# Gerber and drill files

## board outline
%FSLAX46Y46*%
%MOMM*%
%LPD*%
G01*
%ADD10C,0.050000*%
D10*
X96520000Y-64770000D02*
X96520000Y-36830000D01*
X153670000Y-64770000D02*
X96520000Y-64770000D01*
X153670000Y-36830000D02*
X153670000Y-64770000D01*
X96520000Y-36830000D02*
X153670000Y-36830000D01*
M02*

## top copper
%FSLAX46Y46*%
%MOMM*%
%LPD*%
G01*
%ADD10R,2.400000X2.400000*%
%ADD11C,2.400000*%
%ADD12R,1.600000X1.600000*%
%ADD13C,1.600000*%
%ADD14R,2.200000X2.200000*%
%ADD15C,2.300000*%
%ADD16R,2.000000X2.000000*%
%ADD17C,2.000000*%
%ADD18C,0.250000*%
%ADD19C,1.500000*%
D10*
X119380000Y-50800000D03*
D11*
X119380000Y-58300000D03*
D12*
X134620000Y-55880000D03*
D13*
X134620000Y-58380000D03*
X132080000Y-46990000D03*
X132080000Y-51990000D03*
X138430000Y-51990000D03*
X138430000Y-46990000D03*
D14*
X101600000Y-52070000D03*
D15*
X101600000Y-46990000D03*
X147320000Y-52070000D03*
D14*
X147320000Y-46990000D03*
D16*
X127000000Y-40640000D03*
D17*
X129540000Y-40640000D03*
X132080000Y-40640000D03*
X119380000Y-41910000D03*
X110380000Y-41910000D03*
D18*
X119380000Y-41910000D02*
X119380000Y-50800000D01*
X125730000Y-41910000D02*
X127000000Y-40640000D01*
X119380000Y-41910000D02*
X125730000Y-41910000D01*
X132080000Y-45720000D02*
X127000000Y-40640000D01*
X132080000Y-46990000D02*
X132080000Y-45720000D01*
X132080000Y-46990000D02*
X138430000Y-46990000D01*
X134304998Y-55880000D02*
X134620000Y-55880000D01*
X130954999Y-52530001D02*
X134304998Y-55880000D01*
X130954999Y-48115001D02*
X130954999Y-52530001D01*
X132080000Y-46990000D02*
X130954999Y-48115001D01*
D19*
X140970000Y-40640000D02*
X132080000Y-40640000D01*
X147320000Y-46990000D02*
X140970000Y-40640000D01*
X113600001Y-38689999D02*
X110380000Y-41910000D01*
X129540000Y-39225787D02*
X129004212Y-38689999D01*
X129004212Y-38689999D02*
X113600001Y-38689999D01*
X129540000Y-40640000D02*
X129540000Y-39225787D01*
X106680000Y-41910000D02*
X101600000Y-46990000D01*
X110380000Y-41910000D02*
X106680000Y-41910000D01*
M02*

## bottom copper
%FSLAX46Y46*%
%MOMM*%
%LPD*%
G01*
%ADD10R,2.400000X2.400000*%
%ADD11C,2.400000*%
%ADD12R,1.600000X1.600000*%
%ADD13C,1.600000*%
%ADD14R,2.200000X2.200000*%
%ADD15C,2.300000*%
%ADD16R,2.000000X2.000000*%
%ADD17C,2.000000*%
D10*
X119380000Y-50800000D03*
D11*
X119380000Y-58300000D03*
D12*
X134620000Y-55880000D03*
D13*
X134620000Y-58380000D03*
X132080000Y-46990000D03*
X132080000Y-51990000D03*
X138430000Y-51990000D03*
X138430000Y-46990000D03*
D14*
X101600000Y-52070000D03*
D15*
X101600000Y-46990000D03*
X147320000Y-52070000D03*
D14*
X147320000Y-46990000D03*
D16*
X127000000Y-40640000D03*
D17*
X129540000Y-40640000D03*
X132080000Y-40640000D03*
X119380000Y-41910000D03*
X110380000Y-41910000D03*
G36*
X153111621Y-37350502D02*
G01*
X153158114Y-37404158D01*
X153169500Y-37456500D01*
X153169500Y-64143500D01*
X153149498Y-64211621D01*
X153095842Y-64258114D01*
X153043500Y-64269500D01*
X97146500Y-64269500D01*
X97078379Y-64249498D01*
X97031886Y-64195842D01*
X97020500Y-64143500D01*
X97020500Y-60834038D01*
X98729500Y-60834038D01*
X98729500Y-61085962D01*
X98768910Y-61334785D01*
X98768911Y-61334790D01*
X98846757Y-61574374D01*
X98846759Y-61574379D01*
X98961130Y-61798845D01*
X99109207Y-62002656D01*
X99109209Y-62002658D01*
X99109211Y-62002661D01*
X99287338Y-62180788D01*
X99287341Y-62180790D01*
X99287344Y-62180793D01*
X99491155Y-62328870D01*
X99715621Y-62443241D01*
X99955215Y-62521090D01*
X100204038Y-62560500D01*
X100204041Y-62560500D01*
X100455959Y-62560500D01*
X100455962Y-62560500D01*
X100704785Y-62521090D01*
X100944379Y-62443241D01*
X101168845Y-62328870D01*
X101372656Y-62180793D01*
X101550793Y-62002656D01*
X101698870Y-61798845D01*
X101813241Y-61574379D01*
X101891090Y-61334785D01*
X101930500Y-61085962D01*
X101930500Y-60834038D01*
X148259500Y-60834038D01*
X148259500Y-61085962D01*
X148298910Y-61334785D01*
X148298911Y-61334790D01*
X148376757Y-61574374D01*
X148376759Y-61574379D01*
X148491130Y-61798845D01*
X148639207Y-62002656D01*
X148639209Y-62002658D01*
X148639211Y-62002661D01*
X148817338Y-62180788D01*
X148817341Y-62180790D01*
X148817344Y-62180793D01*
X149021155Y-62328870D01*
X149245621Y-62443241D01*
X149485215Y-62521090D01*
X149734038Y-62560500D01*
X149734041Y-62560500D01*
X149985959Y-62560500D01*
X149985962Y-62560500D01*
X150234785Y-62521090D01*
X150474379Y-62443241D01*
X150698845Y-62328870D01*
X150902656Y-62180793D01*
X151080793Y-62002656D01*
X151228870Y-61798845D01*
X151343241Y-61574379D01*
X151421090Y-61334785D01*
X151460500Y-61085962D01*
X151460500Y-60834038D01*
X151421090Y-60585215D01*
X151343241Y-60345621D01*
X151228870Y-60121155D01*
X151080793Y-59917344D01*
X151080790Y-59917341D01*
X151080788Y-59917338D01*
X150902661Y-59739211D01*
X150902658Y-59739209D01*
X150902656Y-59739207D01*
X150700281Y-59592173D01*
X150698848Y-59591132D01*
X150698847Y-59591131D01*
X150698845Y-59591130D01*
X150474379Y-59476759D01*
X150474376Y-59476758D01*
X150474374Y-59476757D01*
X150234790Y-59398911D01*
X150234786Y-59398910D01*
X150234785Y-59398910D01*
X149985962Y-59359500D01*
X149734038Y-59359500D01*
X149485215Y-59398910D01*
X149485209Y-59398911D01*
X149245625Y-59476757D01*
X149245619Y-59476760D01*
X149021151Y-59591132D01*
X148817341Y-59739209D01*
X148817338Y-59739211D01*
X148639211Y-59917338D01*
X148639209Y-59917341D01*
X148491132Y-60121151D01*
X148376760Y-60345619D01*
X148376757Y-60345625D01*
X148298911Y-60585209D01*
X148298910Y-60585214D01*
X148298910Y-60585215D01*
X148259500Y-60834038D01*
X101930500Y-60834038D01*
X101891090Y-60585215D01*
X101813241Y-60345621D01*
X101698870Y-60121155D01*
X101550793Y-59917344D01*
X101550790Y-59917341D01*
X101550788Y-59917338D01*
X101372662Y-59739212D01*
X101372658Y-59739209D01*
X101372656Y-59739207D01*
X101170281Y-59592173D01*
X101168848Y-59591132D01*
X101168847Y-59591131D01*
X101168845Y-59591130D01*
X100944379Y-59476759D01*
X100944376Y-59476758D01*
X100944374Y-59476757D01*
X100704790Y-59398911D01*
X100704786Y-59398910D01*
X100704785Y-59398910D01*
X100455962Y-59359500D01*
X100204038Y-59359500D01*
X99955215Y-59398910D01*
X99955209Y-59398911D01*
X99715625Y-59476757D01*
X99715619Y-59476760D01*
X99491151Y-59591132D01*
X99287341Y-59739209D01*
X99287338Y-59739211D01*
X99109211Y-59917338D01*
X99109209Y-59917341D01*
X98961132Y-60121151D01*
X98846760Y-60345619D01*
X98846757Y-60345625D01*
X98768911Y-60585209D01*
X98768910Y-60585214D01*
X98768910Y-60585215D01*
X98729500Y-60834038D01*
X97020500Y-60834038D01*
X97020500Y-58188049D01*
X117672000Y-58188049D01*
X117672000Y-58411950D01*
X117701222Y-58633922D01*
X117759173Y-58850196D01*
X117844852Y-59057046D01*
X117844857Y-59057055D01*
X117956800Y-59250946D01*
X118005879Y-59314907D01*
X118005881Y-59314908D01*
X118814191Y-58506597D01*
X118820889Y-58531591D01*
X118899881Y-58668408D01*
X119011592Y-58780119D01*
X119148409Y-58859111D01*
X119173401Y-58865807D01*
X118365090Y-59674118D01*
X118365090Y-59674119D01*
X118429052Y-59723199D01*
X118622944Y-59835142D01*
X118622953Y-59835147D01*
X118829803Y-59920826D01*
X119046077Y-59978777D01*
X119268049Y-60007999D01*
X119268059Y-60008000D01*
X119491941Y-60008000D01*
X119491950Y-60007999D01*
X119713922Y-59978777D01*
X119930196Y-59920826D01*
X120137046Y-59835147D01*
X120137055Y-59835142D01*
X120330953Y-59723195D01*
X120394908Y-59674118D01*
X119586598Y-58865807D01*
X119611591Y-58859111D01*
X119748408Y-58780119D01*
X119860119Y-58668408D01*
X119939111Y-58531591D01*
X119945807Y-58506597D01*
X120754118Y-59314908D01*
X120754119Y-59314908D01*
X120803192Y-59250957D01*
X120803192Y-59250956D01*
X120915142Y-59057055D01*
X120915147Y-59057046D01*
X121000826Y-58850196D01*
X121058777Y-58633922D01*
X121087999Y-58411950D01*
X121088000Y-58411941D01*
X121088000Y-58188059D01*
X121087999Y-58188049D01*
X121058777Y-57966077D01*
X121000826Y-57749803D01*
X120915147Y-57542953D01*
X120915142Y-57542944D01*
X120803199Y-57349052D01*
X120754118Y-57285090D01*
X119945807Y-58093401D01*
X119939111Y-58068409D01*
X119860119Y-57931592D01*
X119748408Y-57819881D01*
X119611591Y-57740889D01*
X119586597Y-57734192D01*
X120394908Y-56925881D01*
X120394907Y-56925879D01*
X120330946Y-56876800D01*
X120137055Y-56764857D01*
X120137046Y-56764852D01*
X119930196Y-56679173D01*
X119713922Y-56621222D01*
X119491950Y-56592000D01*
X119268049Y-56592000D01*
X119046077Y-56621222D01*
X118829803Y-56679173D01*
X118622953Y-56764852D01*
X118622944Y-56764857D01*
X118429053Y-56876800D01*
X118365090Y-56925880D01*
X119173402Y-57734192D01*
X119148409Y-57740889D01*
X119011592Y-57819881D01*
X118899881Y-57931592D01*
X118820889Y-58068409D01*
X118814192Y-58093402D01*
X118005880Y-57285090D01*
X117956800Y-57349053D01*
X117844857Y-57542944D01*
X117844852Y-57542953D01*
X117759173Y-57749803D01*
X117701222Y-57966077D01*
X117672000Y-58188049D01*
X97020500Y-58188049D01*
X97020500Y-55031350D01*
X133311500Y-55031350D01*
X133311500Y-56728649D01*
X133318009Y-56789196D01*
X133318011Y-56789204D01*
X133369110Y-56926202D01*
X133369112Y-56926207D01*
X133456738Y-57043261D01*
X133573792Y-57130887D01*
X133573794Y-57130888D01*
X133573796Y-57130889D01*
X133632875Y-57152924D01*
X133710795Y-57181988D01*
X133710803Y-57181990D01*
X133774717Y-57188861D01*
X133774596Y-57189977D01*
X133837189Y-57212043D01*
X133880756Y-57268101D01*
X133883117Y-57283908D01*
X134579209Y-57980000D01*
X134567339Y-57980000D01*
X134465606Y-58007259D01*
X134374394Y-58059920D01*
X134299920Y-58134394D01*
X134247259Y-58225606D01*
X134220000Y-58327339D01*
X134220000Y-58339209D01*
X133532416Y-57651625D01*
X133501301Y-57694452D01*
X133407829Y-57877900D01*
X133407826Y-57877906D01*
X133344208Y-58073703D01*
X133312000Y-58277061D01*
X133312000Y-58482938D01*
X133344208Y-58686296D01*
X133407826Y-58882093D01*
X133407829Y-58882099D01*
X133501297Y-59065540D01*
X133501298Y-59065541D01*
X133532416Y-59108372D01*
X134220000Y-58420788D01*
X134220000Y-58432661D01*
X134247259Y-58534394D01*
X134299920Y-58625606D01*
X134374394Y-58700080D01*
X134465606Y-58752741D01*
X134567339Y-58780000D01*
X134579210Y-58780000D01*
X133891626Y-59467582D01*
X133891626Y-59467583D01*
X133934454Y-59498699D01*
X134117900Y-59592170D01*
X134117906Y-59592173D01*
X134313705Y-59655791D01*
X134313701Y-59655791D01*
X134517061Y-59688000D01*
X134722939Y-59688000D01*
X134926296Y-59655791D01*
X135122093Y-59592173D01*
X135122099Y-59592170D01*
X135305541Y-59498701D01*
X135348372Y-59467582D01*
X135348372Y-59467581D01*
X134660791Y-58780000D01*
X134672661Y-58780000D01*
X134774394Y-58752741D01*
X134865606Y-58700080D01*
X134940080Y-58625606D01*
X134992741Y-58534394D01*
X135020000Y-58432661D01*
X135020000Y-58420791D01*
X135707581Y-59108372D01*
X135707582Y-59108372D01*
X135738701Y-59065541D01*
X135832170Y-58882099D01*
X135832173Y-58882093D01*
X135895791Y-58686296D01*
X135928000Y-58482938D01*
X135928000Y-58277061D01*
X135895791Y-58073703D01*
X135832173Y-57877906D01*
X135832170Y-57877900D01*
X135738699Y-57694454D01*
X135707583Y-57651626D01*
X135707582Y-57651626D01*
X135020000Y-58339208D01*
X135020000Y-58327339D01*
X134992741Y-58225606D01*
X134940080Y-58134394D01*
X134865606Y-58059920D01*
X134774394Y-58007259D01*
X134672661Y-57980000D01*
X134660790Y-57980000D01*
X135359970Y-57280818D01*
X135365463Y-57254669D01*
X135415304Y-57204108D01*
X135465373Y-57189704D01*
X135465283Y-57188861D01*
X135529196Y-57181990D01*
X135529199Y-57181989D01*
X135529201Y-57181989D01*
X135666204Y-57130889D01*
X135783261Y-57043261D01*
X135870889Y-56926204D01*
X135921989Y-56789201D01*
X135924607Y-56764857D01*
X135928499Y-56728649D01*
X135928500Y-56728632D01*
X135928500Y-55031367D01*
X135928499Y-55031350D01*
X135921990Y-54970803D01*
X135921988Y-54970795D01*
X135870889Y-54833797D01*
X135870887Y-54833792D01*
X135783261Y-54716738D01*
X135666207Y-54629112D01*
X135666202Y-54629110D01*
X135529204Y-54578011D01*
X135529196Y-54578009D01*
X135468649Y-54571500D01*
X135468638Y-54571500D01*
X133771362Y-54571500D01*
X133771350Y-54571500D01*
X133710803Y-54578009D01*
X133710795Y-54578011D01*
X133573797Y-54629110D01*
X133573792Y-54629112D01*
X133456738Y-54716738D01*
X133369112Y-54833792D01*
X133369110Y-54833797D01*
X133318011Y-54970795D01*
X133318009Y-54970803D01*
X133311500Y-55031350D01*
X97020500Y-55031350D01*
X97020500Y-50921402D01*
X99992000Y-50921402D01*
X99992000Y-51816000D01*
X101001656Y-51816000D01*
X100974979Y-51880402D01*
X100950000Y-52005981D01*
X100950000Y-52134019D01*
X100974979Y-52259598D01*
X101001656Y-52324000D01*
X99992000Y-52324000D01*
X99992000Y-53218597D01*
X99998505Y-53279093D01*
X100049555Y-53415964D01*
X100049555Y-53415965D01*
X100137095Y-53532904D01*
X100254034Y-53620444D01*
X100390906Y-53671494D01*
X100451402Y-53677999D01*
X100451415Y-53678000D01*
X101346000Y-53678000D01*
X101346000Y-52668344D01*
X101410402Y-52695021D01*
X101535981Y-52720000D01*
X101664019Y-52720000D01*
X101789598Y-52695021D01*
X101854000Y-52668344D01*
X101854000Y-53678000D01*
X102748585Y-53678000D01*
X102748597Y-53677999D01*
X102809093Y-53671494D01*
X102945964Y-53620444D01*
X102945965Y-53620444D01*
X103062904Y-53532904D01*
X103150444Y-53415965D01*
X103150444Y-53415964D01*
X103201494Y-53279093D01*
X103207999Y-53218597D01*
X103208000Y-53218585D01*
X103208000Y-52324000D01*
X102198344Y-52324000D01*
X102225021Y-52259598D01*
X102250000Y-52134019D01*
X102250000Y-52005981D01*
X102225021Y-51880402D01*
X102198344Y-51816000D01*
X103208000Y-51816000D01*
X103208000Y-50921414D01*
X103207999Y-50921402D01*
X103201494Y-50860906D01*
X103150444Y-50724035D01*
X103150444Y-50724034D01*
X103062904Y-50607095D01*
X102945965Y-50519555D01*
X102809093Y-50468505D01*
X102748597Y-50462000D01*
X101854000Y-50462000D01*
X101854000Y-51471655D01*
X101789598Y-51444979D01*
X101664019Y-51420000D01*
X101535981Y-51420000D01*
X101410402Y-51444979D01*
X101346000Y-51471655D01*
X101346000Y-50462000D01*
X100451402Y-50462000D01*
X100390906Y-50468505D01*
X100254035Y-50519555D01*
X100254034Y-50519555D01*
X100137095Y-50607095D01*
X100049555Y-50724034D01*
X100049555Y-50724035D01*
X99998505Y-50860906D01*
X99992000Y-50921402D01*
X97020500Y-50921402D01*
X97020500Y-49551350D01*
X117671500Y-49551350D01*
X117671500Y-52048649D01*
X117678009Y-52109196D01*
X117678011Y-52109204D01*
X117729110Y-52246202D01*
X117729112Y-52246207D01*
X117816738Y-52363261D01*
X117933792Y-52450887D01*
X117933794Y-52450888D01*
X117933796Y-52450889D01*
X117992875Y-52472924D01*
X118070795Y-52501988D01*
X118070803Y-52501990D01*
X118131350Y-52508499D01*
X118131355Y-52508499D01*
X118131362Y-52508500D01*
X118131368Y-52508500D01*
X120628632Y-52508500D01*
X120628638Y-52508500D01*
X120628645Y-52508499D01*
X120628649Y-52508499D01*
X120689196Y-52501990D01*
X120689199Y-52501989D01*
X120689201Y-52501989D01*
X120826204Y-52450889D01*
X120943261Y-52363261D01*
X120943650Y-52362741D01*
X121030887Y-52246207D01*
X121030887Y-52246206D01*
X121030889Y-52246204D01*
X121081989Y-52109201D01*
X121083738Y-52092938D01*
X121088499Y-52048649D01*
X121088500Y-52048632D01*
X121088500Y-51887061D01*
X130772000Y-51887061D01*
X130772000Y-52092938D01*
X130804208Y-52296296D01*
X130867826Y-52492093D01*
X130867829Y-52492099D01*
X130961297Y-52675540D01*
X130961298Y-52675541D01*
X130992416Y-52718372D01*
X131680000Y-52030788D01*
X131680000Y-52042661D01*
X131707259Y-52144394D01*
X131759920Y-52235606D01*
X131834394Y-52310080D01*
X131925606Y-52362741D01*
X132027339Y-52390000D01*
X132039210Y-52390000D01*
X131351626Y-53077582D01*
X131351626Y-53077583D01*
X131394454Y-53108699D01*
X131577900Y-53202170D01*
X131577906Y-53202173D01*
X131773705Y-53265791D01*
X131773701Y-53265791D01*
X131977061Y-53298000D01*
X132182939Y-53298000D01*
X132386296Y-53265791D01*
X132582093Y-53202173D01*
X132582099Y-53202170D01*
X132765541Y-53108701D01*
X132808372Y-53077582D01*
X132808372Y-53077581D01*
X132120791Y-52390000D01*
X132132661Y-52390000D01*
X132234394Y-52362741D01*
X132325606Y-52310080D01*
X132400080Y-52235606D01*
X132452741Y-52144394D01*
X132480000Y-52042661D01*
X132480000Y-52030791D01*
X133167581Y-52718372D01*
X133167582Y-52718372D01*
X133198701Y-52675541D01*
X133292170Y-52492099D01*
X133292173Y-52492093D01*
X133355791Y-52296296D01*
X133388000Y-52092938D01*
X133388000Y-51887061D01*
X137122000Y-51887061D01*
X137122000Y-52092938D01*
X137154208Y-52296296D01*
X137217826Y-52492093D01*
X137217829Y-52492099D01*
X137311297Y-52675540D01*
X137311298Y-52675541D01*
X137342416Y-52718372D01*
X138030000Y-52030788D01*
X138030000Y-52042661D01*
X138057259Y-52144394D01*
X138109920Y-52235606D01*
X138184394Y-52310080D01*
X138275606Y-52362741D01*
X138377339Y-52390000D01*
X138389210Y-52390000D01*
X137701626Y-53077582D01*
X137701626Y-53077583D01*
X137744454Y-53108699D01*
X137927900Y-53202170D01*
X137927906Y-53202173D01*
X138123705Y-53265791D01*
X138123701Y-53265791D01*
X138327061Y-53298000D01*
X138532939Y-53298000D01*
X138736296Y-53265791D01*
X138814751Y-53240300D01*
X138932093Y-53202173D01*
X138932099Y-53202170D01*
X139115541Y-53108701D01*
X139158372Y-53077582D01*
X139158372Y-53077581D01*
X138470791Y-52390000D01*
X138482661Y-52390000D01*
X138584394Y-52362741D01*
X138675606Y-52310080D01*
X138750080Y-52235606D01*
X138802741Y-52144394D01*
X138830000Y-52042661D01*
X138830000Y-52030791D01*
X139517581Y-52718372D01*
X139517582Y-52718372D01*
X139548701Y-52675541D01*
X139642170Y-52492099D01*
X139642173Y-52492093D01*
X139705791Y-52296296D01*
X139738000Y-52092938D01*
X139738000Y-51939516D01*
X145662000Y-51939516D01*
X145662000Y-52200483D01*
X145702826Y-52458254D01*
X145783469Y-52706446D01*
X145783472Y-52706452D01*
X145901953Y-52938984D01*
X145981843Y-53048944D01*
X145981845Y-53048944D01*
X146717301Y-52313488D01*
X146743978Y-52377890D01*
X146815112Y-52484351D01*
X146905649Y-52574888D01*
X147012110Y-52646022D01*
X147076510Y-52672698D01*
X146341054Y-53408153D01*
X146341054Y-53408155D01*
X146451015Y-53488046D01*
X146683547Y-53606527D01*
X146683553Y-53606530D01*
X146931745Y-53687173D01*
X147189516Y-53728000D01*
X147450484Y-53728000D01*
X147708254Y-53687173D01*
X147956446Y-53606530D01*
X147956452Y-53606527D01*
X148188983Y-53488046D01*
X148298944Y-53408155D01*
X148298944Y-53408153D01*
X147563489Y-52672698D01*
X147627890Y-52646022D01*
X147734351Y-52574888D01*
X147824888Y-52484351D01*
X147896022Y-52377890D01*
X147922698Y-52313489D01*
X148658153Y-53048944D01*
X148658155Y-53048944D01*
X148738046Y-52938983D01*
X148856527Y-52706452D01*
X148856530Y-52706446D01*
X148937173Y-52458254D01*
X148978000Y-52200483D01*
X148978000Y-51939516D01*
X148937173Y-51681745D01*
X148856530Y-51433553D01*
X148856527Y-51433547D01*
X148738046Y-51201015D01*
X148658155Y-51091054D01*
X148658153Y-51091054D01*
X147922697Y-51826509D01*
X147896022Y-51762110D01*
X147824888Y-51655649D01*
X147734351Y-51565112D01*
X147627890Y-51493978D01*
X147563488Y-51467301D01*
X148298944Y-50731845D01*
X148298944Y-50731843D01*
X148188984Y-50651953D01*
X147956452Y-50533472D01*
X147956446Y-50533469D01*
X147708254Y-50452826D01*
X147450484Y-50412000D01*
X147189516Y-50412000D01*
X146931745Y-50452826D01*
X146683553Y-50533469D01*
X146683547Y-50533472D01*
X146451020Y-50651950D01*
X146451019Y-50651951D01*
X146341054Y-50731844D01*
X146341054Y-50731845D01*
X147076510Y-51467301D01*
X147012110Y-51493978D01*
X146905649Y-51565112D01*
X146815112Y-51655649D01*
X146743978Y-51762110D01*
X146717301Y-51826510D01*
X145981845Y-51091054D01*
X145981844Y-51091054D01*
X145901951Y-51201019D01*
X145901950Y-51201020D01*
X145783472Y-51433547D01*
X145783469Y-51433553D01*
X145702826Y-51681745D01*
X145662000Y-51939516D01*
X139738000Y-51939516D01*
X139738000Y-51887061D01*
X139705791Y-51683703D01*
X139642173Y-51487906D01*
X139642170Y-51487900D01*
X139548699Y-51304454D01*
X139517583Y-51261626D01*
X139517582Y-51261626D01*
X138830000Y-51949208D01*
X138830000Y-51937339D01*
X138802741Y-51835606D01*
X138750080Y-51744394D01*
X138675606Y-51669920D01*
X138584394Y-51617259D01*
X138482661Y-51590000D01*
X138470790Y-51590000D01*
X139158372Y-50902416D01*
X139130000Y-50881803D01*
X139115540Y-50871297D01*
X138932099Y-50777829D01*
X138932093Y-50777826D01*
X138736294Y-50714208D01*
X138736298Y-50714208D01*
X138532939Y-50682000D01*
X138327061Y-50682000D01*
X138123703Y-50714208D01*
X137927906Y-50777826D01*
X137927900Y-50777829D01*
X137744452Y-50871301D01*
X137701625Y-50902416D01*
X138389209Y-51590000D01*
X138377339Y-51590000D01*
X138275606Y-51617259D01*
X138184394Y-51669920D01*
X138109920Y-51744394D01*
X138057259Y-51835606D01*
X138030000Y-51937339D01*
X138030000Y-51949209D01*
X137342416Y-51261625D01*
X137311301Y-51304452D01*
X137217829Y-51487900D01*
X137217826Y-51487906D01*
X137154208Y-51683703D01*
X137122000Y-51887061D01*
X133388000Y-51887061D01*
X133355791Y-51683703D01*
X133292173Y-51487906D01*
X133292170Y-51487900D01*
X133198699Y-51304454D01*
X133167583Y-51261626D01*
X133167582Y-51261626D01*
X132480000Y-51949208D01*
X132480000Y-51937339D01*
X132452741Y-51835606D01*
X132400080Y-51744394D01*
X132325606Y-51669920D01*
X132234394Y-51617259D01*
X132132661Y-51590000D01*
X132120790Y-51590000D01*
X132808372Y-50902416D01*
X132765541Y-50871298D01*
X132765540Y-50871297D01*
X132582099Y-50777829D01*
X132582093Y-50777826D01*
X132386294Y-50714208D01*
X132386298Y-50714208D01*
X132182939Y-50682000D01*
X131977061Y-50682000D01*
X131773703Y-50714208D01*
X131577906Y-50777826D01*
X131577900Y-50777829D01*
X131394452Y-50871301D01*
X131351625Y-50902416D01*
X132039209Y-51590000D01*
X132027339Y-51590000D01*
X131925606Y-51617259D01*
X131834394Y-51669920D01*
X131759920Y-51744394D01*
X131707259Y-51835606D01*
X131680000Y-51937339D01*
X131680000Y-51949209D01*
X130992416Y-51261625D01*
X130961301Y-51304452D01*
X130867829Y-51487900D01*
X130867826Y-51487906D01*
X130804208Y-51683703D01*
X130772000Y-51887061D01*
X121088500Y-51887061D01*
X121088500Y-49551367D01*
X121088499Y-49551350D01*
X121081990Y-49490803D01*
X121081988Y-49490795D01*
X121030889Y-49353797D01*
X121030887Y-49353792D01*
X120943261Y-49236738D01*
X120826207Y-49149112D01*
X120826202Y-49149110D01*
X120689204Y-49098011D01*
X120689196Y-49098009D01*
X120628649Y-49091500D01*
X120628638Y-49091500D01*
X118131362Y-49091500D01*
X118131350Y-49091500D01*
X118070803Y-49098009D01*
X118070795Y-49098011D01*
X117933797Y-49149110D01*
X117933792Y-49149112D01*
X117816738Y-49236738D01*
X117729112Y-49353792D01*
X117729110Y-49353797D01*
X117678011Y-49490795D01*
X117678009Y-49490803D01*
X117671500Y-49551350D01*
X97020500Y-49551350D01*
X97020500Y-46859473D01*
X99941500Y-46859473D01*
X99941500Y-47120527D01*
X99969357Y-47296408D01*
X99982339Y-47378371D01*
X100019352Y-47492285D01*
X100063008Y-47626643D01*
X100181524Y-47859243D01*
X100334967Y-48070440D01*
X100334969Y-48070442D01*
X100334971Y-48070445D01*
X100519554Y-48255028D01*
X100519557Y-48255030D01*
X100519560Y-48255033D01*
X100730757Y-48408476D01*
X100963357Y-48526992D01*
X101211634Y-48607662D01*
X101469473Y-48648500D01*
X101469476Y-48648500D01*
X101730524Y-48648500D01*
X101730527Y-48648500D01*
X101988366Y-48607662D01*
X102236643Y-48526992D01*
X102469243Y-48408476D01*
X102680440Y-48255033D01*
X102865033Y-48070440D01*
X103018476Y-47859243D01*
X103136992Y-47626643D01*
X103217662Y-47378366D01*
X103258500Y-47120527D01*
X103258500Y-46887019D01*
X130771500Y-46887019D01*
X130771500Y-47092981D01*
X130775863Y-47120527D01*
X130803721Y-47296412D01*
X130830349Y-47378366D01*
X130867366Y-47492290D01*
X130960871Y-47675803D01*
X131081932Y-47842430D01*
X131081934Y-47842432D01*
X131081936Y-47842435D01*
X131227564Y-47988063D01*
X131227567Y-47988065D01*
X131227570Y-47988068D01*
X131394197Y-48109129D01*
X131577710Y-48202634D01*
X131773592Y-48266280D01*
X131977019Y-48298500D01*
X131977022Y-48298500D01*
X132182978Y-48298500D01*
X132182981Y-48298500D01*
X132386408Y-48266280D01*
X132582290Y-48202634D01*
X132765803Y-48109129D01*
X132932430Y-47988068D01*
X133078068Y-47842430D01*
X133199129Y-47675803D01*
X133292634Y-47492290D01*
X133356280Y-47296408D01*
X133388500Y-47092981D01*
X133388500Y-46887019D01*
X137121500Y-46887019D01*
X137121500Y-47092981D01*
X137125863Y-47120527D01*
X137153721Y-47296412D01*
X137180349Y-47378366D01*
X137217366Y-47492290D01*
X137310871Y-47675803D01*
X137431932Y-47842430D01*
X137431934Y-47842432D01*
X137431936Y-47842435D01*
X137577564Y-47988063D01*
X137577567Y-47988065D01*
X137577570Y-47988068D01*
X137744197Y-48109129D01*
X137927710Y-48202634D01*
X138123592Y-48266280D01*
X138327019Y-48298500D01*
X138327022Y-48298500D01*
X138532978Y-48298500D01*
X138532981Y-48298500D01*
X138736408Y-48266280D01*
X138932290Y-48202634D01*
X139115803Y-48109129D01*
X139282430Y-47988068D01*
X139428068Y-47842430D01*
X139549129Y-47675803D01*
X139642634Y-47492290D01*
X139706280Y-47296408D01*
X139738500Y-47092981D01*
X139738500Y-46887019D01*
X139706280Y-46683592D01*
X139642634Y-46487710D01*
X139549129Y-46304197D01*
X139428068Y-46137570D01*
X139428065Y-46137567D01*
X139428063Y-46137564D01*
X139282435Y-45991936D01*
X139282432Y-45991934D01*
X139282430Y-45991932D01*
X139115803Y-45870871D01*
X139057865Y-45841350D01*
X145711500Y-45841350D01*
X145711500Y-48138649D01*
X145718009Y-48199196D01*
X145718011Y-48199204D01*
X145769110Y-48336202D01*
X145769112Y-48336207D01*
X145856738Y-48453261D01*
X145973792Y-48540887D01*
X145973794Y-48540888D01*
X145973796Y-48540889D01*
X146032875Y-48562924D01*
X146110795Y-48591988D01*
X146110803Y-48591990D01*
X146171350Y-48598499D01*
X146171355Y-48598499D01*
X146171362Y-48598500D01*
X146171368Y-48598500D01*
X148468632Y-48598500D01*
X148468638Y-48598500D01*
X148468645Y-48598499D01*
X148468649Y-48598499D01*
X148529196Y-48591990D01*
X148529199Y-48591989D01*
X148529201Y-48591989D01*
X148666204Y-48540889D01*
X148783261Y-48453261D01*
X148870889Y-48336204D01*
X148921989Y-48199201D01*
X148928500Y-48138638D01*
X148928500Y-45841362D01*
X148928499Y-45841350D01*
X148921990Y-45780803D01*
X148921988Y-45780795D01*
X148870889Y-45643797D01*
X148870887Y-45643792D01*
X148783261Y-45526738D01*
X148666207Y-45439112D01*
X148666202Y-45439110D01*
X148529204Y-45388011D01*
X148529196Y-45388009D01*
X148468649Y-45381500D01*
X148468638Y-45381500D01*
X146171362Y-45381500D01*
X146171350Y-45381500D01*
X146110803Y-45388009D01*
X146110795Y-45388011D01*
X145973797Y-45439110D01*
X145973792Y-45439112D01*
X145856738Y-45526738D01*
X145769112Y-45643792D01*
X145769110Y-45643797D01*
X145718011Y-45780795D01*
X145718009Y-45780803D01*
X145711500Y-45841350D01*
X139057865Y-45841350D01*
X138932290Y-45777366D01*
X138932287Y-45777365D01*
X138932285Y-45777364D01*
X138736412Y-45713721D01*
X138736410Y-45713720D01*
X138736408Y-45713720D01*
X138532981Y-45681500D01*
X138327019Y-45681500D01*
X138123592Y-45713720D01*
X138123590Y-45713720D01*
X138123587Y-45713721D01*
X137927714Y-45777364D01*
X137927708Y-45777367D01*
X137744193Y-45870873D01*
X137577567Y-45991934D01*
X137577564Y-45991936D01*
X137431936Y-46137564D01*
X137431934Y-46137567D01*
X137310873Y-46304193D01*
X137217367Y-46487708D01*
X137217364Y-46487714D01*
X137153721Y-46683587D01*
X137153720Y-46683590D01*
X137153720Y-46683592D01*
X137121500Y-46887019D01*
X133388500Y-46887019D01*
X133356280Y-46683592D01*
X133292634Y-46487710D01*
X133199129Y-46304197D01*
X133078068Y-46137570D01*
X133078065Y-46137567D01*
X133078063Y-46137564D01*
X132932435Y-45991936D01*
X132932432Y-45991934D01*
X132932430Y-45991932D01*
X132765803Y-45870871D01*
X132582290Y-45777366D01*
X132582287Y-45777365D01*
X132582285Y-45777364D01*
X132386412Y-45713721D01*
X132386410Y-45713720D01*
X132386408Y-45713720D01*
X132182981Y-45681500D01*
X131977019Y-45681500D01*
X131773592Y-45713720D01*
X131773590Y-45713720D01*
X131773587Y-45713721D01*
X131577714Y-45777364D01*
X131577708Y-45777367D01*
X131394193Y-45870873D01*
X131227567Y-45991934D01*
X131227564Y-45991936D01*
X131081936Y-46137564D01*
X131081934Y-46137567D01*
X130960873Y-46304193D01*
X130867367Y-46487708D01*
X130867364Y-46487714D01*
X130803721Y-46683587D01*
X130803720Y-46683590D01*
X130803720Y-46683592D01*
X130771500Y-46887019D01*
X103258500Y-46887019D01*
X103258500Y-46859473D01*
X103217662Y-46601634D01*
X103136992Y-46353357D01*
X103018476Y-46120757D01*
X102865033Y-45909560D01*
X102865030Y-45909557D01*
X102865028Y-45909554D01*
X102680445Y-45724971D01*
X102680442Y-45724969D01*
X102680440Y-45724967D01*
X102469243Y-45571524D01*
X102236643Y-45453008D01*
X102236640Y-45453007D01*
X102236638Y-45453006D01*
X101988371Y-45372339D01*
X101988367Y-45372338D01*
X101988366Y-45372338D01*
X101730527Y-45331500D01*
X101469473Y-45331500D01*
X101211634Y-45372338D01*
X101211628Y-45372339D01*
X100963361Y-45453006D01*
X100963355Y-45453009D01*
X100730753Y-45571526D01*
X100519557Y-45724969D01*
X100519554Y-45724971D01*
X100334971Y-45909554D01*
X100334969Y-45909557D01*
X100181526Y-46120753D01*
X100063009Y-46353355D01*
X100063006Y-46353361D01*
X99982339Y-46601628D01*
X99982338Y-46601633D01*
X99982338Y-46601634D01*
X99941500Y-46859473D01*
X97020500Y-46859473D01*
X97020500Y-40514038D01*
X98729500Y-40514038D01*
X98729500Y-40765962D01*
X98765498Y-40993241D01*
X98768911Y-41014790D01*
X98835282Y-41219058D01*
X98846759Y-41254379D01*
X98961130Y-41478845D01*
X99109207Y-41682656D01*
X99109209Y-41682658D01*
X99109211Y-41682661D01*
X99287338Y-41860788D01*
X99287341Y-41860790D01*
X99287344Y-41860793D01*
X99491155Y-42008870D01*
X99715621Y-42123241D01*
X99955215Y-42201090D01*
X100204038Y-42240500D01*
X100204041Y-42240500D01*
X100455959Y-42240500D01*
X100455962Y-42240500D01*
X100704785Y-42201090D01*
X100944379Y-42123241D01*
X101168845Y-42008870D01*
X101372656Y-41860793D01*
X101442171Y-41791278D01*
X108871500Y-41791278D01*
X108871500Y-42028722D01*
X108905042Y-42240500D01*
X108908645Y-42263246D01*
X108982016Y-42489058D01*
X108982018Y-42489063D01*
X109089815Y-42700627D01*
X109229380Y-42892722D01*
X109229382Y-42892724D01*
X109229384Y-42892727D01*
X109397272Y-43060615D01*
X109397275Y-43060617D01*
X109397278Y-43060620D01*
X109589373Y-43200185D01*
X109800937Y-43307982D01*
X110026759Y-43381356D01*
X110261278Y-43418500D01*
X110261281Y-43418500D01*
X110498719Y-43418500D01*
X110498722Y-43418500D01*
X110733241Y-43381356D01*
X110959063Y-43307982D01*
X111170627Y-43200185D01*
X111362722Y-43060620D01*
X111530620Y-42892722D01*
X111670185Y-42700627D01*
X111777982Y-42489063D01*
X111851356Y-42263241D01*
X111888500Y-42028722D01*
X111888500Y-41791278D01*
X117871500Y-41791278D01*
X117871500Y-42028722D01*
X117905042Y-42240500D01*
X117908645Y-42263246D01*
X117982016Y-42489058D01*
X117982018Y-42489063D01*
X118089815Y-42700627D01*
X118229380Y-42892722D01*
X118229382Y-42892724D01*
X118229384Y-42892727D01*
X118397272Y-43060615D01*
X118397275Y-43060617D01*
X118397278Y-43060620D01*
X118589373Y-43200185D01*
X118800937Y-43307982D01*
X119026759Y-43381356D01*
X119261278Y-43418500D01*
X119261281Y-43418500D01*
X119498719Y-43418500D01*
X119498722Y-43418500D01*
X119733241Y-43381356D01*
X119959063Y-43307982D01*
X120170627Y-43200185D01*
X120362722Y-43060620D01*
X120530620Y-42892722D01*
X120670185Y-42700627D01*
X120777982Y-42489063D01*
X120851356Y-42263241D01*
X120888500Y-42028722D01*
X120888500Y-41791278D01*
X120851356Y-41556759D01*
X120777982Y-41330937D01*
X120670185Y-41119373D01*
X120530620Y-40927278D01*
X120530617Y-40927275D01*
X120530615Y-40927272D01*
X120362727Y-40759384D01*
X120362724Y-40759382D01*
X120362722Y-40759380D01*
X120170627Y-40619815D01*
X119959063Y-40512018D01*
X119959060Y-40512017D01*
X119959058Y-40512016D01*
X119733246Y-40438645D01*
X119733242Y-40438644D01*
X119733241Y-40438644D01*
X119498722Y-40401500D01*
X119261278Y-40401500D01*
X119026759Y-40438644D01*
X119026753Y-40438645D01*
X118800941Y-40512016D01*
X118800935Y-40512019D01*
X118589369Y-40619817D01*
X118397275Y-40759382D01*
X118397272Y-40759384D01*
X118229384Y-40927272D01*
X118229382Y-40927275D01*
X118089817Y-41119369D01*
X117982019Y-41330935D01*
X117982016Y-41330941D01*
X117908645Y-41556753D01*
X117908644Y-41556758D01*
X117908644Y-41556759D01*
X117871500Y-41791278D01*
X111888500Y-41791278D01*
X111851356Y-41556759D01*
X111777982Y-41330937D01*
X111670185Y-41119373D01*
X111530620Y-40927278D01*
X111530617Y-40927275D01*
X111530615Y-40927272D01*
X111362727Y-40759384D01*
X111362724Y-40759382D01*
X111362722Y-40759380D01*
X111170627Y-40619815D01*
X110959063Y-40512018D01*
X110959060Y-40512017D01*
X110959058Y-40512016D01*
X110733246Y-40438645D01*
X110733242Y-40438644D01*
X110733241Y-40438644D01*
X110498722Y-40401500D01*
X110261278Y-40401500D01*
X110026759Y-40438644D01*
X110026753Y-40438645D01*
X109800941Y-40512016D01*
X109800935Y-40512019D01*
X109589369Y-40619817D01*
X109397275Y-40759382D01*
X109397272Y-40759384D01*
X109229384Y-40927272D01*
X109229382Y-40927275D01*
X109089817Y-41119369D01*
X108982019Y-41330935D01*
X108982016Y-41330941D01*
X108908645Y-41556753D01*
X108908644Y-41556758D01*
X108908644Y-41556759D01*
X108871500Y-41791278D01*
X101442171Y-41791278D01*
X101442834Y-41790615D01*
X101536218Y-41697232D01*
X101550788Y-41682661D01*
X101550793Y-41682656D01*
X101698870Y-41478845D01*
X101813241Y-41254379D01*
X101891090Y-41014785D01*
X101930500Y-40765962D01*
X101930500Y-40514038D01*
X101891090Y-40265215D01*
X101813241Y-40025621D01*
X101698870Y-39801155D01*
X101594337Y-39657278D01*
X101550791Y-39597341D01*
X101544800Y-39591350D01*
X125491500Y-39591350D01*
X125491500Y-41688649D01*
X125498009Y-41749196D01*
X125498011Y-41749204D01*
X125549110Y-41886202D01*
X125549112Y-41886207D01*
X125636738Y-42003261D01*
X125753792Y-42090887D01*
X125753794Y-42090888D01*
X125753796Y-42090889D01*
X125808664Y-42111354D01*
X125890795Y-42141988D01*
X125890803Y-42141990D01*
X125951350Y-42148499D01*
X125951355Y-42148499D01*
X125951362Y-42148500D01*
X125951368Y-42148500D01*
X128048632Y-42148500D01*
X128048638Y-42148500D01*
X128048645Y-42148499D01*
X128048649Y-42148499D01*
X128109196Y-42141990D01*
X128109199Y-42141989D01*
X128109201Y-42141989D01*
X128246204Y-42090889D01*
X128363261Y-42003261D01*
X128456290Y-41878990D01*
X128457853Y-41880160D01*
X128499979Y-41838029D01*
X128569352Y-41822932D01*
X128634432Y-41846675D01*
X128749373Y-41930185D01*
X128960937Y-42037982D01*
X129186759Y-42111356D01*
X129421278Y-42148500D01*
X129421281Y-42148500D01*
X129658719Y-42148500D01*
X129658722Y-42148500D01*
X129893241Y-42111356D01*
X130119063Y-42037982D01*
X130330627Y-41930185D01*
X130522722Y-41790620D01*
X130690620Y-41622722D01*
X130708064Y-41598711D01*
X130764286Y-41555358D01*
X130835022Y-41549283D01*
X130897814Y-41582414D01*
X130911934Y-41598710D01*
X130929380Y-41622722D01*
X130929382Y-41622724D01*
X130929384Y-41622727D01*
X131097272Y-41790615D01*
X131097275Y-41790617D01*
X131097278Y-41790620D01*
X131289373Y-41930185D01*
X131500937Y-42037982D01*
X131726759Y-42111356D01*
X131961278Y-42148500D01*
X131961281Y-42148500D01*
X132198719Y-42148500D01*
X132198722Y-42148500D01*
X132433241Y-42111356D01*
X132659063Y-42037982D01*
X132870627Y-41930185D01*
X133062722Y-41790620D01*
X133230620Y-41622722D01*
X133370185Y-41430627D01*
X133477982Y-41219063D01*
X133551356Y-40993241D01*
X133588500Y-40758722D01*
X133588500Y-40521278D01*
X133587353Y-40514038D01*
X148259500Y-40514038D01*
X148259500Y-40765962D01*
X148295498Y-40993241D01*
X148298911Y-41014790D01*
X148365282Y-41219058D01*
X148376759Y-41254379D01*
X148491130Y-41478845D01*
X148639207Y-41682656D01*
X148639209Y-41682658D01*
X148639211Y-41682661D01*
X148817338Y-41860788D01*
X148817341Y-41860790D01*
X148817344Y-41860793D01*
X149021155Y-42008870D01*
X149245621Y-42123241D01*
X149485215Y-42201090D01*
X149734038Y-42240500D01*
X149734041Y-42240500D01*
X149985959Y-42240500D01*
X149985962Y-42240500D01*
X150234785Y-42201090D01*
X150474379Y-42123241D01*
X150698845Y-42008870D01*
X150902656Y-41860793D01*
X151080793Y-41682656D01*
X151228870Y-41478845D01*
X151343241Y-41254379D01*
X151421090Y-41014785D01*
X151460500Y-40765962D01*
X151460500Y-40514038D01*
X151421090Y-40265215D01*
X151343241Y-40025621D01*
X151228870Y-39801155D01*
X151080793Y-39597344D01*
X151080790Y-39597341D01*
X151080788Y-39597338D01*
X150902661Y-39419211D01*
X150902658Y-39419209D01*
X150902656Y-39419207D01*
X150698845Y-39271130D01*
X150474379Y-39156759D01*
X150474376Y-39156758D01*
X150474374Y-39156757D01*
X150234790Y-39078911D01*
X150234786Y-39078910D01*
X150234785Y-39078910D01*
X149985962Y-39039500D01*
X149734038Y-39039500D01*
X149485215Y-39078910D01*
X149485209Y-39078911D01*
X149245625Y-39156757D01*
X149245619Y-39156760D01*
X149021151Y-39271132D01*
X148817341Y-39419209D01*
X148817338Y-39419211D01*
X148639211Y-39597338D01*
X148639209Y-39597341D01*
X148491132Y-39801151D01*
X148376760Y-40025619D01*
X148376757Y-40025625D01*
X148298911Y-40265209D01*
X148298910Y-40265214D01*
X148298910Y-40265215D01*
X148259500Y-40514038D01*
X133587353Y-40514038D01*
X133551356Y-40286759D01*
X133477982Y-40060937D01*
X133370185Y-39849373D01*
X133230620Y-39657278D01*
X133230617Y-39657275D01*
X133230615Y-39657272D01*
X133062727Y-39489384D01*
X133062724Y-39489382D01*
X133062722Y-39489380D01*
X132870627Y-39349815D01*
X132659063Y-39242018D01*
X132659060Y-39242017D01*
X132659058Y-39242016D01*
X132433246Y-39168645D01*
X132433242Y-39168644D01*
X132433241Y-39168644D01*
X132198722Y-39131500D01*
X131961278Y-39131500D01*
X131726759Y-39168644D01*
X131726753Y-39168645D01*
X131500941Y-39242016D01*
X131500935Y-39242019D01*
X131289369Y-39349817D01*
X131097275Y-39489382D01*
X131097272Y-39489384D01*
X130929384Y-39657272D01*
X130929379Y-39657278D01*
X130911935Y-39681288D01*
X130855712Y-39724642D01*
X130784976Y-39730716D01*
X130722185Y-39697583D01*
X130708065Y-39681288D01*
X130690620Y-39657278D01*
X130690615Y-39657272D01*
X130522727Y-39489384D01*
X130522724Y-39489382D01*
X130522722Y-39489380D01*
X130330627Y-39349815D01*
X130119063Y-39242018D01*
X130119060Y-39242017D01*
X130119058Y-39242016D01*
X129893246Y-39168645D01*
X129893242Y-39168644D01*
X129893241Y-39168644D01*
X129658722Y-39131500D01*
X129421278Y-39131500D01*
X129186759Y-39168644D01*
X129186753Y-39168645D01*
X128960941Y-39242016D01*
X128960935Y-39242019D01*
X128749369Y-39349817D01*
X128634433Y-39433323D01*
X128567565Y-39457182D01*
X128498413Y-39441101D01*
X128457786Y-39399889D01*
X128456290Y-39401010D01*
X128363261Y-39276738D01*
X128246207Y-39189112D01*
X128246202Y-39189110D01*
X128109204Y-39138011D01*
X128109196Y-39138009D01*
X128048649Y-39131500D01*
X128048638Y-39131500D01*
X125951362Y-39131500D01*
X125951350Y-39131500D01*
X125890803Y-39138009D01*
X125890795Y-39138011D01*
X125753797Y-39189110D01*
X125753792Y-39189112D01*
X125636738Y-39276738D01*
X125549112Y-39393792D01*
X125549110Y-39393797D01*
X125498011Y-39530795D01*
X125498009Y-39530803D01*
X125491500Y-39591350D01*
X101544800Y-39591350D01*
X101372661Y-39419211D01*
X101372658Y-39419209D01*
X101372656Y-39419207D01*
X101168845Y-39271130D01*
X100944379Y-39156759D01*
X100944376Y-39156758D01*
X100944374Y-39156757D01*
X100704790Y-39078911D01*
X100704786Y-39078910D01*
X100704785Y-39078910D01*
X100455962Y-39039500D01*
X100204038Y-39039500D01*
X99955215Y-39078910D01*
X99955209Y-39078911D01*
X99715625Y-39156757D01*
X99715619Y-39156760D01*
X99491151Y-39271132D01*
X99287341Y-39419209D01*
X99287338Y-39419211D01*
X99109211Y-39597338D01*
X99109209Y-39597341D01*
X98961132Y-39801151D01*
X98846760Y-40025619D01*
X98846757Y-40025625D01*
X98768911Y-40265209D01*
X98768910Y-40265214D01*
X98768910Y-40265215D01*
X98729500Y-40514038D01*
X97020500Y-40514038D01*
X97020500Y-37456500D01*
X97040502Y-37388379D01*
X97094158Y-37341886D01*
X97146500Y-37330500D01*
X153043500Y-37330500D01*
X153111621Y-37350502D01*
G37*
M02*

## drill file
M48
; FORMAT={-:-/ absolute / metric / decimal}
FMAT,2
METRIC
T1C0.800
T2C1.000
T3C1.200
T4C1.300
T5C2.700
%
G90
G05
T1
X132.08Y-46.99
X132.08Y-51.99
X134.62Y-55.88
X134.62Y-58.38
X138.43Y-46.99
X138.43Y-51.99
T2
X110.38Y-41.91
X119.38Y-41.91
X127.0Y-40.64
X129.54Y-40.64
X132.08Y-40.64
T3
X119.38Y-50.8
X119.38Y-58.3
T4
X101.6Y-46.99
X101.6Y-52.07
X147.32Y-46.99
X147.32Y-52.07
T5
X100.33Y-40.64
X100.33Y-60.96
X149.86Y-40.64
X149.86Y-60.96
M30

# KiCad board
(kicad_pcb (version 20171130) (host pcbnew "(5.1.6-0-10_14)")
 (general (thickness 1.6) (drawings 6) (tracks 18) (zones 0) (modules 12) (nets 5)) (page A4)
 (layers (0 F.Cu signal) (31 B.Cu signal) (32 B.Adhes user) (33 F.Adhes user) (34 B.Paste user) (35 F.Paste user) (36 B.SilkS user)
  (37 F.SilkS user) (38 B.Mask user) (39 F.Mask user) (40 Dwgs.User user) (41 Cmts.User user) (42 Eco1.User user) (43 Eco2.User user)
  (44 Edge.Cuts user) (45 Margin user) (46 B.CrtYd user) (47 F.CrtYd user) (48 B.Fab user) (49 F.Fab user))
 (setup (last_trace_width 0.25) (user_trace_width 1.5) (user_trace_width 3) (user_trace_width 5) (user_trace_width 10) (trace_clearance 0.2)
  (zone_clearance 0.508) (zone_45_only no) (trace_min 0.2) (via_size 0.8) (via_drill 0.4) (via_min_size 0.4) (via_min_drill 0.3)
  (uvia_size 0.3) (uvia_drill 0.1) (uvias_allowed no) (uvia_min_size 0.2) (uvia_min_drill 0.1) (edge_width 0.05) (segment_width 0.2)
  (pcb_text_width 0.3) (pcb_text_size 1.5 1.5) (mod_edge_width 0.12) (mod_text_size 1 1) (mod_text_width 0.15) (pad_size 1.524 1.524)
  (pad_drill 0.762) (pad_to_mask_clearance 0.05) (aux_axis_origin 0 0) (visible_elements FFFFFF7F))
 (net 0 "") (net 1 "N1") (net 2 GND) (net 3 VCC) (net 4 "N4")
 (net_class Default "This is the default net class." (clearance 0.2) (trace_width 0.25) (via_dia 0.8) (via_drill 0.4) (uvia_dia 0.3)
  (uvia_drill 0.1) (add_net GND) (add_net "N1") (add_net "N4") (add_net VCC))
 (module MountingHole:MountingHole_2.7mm (layer F.Cu) (at 149.86 60.96)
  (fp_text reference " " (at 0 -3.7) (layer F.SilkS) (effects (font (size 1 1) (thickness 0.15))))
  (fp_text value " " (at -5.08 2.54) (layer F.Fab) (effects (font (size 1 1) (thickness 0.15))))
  (pad 1 np_thru_hole circle (at 0 0) (size 2.7 2.7) (drill 2.7) (layers *.Cu *.Mask)))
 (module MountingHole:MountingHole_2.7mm (layer F.Cu) (at 149.86 40.64)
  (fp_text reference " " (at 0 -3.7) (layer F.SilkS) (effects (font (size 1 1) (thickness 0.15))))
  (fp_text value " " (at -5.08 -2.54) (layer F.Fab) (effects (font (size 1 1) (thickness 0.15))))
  (pad 1 np_thru_hole circle (at 0 0) (size 2.7 2.7) (drill 2.7) (layers *.Cu *.Mask)))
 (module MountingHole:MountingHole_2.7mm (layer F.Cu) (at 100.33 60.96)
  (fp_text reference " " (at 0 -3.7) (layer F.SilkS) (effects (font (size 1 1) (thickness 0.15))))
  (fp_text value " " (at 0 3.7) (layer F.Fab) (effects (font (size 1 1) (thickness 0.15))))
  (pad 1 np_thru_hole circle (at 0 0) (size 2.7 2.7) (drill 2.7) (layers *.Cu *.Mask)))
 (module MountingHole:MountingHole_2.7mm (layer F.Cu) (at 100.33 40.64)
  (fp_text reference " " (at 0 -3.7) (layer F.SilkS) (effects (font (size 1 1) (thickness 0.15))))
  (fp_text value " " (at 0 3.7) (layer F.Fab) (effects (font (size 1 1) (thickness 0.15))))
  (pad 1 np_thru_hole circle (at 0 0) (size 2.7 2.7) (drill 2.7) (layers *.Cu *.Mask)))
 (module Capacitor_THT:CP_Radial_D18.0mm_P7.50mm (layer F.Cu) (at 119.38 50.8 270)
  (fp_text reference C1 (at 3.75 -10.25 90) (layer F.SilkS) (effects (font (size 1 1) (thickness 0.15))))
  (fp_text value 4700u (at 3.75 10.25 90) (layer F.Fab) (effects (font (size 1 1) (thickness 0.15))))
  (pad 1 thru_hole rect (at 0 0 270) (size 2.4 2.4) (drill 1.2) (layers *.Cu *.Mask) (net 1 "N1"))
  (pad 2 thru_hole circle (at 7.5 0 270) (size 2.4 2.4) (drill 1.2) (layers *.Cu *.Mask) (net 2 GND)))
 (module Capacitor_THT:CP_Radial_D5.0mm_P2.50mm (layer F.Cu) (at 134.62 55.88 270)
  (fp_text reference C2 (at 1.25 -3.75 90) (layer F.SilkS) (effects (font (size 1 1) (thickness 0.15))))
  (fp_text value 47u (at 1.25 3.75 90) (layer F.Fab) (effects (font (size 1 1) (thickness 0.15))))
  (pad 1 thru_hole rect (at 0 0 270) (size 1.6 1.6) (drill 0.8) (layers *.Cu *.Mask) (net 1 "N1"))
  (pad 2 thru_hole circle (at 2.5 0 270) (size 1.6 1.6) (drill 0.8) (layers *.Cu *.Mask) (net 2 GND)))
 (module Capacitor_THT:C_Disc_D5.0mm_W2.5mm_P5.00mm (layer F.Cu) (at 132.08 46.99 270)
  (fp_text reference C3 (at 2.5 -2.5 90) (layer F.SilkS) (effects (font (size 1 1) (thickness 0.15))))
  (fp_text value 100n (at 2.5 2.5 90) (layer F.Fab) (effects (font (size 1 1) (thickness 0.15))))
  (pad 1 thru_hole circle (at 0 0 270) (size 1.6 1.6) (drill 0.8) (layers *.Cu *.Mask) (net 1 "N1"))
  (pad 2 thru_hole circle (at 5 0 270) (size 1.6 1.6) (drill 0.8) (layers *.Cu *.Mask) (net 2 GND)))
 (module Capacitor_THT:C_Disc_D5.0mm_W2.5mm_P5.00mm (layer F.Cu) (at 138.43 46.99 270)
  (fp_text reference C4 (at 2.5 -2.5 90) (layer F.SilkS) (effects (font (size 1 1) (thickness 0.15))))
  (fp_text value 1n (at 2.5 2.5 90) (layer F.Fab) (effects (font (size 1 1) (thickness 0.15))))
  (pad 2 thru_hole circle (at 5 0 270) (size 1.6 1.6) (drill 0.8) (layers *.Cu *.Mask) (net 2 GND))
  (pad 1 thru_hole circle (at 0 0 270) (size 1.6 1.6) (drill 0.8) (layers *.Cu *.Mask) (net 1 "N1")))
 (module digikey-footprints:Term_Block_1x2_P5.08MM (layer F.Cu) (at 101.6 52.07 90)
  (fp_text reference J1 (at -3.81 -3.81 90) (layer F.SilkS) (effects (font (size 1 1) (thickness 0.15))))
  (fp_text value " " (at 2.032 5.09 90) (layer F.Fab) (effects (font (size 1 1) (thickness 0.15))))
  (pad 1 thru_hole rect (at 0 0 90) (size 2.2 2.2) (drill 1.3) (layers *.Cu *.Mask) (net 2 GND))
  (pad 2 thru_hole circle (at 5.08 0 90) (size 2.3 2.3) (drill 1.3) (layers *.Cu *.Mask) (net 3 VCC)))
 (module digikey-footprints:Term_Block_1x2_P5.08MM (layer F.Cu) (at 147.32 46.99 270)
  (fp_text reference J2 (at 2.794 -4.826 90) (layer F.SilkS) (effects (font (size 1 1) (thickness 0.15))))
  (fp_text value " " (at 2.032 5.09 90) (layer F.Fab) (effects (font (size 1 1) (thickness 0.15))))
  (pad 2 thru_hole circle (at 5.08 0 270) (size 2.3 2.3) (drill 1.3) (layers *.Cu *.Mask) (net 2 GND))
  (pad 1 thru_hole rect (at 0 0 270) (size 2.2 2.2) (drill 1.3) (layers *.Cu *.Mask) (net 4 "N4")))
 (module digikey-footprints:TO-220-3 (layer F.Cu) (at 127 40.64)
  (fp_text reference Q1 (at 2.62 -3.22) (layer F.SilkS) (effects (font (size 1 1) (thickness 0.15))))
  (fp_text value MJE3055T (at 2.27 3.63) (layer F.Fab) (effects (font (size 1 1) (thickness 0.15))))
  (pad 1 thru_hole rect (at 0 0) (size 2 2) (drill 1) (layers *.Cu *.Mask) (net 1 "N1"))
  (pad 2 thru_hole circle (at 2.54 0) (size 2 2) (drill 1) (layers *.Cu *.Mask) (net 3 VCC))
  (pad 3 thru_hole circle (at 5.08 0) (size 2 2) (drill 1) (layers *.Cu *.Mask) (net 4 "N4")))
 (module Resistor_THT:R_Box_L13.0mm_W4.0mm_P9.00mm (layer F.Cu) (at 119.38 41.91 180)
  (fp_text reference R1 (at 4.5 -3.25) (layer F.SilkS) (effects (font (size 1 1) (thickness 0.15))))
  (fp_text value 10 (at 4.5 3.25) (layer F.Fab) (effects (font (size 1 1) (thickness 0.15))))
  (pad 1 thru_hole circle (at 0 0 180) (size 2 2) (drill 1) (layers *.Cu *.Mask) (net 1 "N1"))
  (pad 2 thru_hole circle (at 9 0 180) (size 2 2) (drill 1) (layers *.Cu *.Mask) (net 3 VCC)))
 (gr_line (start 96.52 64.77) (end 96.52 36.83) (layer Edge.Cuts) (width 0.05))
 (gr_line (start 153.67 64.77) (end 96.52 64.77) (layer Edge.Cuts) (width 0.05))
 (gr_line (start 153.67 36.83) (end 153.67 64.77) (layer Edge.Cuts) (width 0.05))
 (gr_line (start 96.52 36.83) (end 153.67 36.83) (layer Edge.Cuts) (width 0.05))
 (segment (start 119.38 41.91) (end 119.38 50.8) (width 0.25) (layer F.Cu) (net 1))
 (segment (start 125.73 41.91) (end 127 40.64) (width 0.25) (layer F.Cu) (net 1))
 (segment (start 119.38 41.91) (end 125.73 41.91) (width 0.25) (layer F.Cu) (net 1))
 (segment (start 132.08 45.72) (end 127 40.64) (width 0.25) (layer F.Cu) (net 1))
 (segment (start 132.08 46.99) (end 132.08 45.72) (width 0.25) (layer F.Cu) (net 1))
 (segment (start 132.08 46.99) (end 138.43 46.99) (width 0.25) (layer F.Cu) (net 1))
 (segment (start 134.304998 55.88) (end 134.62 55.88) (width 0.25) (layer F.Cu) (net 1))
 (segment (start 130.954999 52.530001) (end 134.304998 55.88) (width 0.25) (layer F.Cu) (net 1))
 (segment (start 130.954999 48.115001) (end 130.954999 52.530001) (width 0.25) (layer F.Cu) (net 1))
 (segment (start 132.08 46.99) (end 130.954999 48.115001) (width 0.25) (layer F.Cu) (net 1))
 (segment (start 140.97 40.64) (end 132.08 40.64) (width 1.5) (layer F.Cu) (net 4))
 (segment (start 147.32 46.99) (end 140.97 40.64) (width 1.5) (layer F.Cu) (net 4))
 (segment (start 113.600001 38.689999) (end 110.38 41.91) (width 1.5) (layer F.Cu) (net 3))
 (segment (start 129.54 39.225787) (end 129.004212 38.689999) (width 1.5) (layer F.Cu) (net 3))
 (segment (start 129.004212 38.689999) (end 113.600001 38.689999) (width 1.5) (layer F.Cu) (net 3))
 (segment (start 129.54 40.64) (end 129.54 39.225787) (width 1.5) (layer F.Cu) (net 3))
 (segment (start 106.68 41.91) (end 101.6 46.99) (width 1.5) (layer F.Cu) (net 3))
 (segment (start 110.38 41.91) (end 106.68 41.91) (width 1.5) (layer F.Cu) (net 3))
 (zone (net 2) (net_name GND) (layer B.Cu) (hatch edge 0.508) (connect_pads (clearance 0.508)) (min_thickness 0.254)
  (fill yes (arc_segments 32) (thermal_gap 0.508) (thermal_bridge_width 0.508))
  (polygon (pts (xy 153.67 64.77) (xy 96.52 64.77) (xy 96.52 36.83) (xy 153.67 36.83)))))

